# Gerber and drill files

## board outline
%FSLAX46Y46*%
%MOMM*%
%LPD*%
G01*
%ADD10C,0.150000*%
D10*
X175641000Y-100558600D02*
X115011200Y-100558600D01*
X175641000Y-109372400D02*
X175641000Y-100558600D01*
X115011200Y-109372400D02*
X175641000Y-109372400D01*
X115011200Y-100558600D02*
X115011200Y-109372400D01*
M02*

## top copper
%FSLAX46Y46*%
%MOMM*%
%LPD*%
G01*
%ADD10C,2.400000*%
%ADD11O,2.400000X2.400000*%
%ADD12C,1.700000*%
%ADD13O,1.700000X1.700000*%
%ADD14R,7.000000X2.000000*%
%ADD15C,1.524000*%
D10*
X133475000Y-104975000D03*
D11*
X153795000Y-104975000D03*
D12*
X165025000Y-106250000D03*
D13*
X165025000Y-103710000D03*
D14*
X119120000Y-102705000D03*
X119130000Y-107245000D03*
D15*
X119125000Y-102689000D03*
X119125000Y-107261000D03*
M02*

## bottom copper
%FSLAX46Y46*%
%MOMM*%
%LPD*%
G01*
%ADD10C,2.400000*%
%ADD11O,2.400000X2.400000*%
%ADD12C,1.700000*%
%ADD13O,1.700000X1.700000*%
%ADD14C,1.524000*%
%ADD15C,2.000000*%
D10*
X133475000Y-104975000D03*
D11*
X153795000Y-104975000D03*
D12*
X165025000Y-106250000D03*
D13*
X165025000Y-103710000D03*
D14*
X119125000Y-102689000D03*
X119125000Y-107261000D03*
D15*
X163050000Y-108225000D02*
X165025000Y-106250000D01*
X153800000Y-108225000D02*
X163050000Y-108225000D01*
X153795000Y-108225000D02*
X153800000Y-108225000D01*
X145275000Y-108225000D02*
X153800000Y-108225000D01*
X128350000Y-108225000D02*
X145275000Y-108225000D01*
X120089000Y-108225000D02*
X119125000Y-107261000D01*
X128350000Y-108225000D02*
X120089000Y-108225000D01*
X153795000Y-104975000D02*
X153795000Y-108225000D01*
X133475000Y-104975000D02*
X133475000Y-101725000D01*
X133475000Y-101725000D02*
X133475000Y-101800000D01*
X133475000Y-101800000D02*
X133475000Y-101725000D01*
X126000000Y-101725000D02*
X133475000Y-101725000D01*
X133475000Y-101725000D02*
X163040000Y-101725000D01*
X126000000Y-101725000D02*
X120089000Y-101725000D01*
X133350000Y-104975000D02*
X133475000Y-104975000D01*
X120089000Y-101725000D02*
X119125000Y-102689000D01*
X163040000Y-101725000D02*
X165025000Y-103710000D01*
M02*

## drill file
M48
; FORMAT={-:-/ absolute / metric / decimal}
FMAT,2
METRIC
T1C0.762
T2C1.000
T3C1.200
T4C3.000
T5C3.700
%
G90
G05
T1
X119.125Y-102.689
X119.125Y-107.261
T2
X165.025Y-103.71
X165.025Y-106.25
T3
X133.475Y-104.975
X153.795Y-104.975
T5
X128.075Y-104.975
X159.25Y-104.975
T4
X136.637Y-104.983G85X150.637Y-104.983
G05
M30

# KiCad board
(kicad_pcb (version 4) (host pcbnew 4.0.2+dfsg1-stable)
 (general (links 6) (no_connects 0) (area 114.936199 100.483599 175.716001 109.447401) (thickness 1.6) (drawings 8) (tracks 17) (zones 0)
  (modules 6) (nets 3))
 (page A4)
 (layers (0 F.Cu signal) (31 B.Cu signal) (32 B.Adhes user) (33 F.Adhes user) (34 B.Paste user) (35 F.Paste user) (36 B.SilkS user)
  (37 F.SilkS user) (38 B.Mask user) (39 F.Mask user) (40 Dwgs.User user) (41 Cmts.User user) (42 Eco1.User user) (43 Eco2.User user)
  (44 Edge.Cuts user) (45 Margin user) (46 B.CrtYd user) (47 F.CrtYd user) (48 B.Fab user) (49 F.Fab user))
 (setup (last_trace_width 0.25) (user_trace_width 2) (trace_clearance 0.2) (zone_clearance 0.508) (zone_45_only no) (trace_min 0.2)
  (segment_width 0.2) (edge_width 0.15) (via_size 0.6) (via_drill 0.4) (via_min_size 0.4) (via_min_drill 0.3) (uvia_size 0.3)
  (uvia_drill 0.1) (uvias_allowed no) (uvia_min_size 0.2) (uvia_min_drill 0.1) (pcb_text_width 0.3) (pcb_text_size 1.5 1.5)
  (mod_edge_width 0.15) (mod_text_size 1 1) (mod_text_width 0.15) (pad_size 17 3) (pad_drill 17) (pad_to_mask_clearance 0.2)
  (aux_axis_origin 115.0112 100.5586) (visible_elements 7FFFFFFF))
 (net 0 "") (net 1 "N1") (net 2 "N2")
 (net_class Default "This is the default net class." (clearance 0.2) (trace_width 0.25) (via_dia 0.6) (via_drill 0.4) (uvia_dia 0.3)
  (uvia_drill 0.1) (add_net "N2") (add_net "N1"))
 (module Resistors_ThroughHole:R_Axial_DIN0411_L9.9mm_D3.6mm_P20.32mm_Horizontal (layer F.Cu) (at 133.475 104.975)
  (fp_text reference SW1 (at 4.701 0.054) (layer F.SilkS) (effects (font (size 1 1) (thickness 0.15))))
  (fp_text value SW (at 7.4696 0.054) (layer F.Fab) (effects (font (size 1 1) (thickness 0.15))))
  (pad 1 thru_hole circle (at 0 0) (size 2.4 2.4) (drill 1.2) (layers *.Cu *.Mask) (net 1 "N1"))
  (pad 2 thru_hole oval (at 20.32 0) (size 2.4 2.4) (drill 1.2) (layers *.Cu *.Mask) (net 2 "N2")))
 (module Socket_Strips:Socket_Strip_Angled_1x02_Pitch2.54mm (layer F.Cu) (at 165.025 106.25 180)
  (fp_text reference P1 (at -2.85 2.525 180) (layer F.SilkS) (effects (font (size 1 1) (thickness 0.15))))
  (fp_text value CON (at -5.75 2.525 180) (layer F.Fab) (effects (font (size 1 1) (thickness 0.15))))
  (pad 1 thru_hole circle (at 0 0 180) (size 1.7 1.7) (drill 1) (layers *.Cu *.Mask) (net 2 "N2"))
  (pad 2 thru_hole oval (at 0 2.54 180) (size 1.7 1.7) (drill 1) (layers *.Cu *.Mask) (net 1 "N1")))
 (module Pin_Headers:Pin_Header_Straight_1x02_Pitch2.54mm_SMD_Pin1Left (layer F.Cu) (at 119.125 104.975)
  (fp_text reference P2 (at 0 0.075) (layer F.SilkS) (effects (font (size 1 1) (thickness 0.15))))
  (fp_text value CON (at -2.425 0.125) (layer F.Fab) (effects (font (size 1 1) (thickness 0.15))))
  (pad 1 smd rect (at -1.655 -1.27) (size 7 2) (drill (offset 1.65 -1)) (layers F.Cu F.Paste F.Mask) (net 1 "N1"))
  (pad 2 smd rect (at 1.655 1.27) (size 7 2) (drill (offset -1.65 1)) (layers F.Cu F.Paste F.Mask) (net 2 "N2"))
  (pad 1 thru_hole circle (at 0 -2.286) (size 1.524 1.524) (drill 0.762) (layers *.Cu *.Mask) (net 1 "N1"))
  (pad 2 thru_hole circle (at 0 2.286) (size 1.524 1.524) (drill 0.762) (layers *.Cu *.Mask) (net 2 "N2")))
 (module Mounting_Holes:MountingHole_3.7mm (layer F.Cu) (at 159.25 104.975)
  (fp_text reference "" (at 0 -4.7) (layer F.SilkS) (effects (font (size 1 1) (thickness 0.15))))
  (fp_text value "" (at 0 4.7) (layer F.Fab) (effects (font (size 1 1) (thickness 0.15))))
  (pad 1 np_thru_hole circle (at 0 0) (size 3.7 3.7) (drill 3.7) (layers *.Cu *.Mask)))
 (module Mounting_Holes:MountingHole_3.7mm (layer F.Cu) (at 128.075 104.975)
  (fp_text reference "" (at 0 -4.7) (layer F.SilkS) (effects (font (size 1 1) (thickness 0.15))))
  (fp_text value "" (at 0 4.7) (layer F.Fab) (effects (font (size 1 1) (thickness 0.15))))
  (pad 1 np_thru_hole circle (at 0 0) (size 3.7 3.7) (drill 3.7) (layers *.Cu *.Mask)))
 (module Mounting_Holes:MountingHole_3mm (layer F.Cu) (at 146.4116 105.2082) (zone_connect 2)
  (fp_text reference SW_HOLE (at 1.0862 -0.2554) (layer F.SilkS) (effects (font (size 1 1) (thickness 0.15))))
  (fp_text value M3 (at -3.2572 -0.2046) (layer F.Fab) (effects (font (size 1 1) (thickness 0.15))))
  (pad "" np_thru_hole oval (at -2.775 -0.225) (size 17 3) (drill oval 17 3) (layers *.Cu *.Mask) (zone_connect 2)))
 (gr_line (start 175.641 100.5586) (end 115.0112 100.5586) (angle 90) (layer Edge.Cuts) (width 0.15))
 (gr_line (start 175.641 109.3724) (end 175.641 100.5586) (angle 90) (layer Edge.Cuts) (width 0.15))
 (gr_line (start 115.0112 109.3724) (end 175.641 109.3724) (angle 90) (layer Edge.Cuts) (width 0.15))
 (gr_line (start 115.0112 100.5586) (end 115.0112 109.3724) (angle 90) (layer Edge.Cuts) (width 0.15))
 (segment (start 163.05 108.225) (end 165.025 106.25) (width 2) (layer B.Cu) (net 2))
 (segment (start 153.8 108.225) (end 163.05 108.225) (width 2) (layer B.Cu) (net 2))
 (segment (start 153.795 108.225) (end 153.8 108.225) (width 2) (layer B.Cu) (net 2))
 (segment (start 145.275 108.225) (end 153.8 108.225) (width 2) (layer B.Cu) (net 2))
 (segment (start 128.35 108.225) (end 145.275 108.225) (width 2) (layer B.Cu) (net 2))
 (segment (start 120.089 108.225) (end 119.125 107.261) (width 2) (layer B.Cu) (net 2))
 (segment (start 128.35 108.225) (end 120.089 108.225) (width 2) (layer B.Cu) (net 2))
 (segment (start 153.795 104.975) (end 153.795 108.225) (width 2) (layer B.Cu) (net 2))
 (segment (start 133.475 104.975) (end 133.475 101.725) (width 2) (layer B.Cu) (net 1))
 (segment (start 133.475 101.725) (end 133.475 101.8) (width 2) (layer B.Cu) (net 1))
 (segment (start 133.475 101.8) (end 133.475 101.725) (width 2) (layer B.Cu) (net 1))
 (segment (start 126 101.725) (end 133.475 101.725) (width 2) (layer B.Cu) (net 1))
 (segment (start 133.475 101.725) (end 163.04 101.725) (width 2) (layer B.Cu) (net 1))
 (segment (start 126 101.725) (end 120.089 101.725) (width 2) (layer B.Cu) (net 1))
 (segment (start 133.35 104.975) (end 133.475 104.975) (width 2) (layer B.Cu) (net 1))
 (segment (start 120.089 101.725) (end 119.125 102.689) (width 2) (layer B.Cu) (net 1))
 (segment (start 163.04 101.725) (end 165.025 103.71) (width 2) (layer B.Cu) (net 1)))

